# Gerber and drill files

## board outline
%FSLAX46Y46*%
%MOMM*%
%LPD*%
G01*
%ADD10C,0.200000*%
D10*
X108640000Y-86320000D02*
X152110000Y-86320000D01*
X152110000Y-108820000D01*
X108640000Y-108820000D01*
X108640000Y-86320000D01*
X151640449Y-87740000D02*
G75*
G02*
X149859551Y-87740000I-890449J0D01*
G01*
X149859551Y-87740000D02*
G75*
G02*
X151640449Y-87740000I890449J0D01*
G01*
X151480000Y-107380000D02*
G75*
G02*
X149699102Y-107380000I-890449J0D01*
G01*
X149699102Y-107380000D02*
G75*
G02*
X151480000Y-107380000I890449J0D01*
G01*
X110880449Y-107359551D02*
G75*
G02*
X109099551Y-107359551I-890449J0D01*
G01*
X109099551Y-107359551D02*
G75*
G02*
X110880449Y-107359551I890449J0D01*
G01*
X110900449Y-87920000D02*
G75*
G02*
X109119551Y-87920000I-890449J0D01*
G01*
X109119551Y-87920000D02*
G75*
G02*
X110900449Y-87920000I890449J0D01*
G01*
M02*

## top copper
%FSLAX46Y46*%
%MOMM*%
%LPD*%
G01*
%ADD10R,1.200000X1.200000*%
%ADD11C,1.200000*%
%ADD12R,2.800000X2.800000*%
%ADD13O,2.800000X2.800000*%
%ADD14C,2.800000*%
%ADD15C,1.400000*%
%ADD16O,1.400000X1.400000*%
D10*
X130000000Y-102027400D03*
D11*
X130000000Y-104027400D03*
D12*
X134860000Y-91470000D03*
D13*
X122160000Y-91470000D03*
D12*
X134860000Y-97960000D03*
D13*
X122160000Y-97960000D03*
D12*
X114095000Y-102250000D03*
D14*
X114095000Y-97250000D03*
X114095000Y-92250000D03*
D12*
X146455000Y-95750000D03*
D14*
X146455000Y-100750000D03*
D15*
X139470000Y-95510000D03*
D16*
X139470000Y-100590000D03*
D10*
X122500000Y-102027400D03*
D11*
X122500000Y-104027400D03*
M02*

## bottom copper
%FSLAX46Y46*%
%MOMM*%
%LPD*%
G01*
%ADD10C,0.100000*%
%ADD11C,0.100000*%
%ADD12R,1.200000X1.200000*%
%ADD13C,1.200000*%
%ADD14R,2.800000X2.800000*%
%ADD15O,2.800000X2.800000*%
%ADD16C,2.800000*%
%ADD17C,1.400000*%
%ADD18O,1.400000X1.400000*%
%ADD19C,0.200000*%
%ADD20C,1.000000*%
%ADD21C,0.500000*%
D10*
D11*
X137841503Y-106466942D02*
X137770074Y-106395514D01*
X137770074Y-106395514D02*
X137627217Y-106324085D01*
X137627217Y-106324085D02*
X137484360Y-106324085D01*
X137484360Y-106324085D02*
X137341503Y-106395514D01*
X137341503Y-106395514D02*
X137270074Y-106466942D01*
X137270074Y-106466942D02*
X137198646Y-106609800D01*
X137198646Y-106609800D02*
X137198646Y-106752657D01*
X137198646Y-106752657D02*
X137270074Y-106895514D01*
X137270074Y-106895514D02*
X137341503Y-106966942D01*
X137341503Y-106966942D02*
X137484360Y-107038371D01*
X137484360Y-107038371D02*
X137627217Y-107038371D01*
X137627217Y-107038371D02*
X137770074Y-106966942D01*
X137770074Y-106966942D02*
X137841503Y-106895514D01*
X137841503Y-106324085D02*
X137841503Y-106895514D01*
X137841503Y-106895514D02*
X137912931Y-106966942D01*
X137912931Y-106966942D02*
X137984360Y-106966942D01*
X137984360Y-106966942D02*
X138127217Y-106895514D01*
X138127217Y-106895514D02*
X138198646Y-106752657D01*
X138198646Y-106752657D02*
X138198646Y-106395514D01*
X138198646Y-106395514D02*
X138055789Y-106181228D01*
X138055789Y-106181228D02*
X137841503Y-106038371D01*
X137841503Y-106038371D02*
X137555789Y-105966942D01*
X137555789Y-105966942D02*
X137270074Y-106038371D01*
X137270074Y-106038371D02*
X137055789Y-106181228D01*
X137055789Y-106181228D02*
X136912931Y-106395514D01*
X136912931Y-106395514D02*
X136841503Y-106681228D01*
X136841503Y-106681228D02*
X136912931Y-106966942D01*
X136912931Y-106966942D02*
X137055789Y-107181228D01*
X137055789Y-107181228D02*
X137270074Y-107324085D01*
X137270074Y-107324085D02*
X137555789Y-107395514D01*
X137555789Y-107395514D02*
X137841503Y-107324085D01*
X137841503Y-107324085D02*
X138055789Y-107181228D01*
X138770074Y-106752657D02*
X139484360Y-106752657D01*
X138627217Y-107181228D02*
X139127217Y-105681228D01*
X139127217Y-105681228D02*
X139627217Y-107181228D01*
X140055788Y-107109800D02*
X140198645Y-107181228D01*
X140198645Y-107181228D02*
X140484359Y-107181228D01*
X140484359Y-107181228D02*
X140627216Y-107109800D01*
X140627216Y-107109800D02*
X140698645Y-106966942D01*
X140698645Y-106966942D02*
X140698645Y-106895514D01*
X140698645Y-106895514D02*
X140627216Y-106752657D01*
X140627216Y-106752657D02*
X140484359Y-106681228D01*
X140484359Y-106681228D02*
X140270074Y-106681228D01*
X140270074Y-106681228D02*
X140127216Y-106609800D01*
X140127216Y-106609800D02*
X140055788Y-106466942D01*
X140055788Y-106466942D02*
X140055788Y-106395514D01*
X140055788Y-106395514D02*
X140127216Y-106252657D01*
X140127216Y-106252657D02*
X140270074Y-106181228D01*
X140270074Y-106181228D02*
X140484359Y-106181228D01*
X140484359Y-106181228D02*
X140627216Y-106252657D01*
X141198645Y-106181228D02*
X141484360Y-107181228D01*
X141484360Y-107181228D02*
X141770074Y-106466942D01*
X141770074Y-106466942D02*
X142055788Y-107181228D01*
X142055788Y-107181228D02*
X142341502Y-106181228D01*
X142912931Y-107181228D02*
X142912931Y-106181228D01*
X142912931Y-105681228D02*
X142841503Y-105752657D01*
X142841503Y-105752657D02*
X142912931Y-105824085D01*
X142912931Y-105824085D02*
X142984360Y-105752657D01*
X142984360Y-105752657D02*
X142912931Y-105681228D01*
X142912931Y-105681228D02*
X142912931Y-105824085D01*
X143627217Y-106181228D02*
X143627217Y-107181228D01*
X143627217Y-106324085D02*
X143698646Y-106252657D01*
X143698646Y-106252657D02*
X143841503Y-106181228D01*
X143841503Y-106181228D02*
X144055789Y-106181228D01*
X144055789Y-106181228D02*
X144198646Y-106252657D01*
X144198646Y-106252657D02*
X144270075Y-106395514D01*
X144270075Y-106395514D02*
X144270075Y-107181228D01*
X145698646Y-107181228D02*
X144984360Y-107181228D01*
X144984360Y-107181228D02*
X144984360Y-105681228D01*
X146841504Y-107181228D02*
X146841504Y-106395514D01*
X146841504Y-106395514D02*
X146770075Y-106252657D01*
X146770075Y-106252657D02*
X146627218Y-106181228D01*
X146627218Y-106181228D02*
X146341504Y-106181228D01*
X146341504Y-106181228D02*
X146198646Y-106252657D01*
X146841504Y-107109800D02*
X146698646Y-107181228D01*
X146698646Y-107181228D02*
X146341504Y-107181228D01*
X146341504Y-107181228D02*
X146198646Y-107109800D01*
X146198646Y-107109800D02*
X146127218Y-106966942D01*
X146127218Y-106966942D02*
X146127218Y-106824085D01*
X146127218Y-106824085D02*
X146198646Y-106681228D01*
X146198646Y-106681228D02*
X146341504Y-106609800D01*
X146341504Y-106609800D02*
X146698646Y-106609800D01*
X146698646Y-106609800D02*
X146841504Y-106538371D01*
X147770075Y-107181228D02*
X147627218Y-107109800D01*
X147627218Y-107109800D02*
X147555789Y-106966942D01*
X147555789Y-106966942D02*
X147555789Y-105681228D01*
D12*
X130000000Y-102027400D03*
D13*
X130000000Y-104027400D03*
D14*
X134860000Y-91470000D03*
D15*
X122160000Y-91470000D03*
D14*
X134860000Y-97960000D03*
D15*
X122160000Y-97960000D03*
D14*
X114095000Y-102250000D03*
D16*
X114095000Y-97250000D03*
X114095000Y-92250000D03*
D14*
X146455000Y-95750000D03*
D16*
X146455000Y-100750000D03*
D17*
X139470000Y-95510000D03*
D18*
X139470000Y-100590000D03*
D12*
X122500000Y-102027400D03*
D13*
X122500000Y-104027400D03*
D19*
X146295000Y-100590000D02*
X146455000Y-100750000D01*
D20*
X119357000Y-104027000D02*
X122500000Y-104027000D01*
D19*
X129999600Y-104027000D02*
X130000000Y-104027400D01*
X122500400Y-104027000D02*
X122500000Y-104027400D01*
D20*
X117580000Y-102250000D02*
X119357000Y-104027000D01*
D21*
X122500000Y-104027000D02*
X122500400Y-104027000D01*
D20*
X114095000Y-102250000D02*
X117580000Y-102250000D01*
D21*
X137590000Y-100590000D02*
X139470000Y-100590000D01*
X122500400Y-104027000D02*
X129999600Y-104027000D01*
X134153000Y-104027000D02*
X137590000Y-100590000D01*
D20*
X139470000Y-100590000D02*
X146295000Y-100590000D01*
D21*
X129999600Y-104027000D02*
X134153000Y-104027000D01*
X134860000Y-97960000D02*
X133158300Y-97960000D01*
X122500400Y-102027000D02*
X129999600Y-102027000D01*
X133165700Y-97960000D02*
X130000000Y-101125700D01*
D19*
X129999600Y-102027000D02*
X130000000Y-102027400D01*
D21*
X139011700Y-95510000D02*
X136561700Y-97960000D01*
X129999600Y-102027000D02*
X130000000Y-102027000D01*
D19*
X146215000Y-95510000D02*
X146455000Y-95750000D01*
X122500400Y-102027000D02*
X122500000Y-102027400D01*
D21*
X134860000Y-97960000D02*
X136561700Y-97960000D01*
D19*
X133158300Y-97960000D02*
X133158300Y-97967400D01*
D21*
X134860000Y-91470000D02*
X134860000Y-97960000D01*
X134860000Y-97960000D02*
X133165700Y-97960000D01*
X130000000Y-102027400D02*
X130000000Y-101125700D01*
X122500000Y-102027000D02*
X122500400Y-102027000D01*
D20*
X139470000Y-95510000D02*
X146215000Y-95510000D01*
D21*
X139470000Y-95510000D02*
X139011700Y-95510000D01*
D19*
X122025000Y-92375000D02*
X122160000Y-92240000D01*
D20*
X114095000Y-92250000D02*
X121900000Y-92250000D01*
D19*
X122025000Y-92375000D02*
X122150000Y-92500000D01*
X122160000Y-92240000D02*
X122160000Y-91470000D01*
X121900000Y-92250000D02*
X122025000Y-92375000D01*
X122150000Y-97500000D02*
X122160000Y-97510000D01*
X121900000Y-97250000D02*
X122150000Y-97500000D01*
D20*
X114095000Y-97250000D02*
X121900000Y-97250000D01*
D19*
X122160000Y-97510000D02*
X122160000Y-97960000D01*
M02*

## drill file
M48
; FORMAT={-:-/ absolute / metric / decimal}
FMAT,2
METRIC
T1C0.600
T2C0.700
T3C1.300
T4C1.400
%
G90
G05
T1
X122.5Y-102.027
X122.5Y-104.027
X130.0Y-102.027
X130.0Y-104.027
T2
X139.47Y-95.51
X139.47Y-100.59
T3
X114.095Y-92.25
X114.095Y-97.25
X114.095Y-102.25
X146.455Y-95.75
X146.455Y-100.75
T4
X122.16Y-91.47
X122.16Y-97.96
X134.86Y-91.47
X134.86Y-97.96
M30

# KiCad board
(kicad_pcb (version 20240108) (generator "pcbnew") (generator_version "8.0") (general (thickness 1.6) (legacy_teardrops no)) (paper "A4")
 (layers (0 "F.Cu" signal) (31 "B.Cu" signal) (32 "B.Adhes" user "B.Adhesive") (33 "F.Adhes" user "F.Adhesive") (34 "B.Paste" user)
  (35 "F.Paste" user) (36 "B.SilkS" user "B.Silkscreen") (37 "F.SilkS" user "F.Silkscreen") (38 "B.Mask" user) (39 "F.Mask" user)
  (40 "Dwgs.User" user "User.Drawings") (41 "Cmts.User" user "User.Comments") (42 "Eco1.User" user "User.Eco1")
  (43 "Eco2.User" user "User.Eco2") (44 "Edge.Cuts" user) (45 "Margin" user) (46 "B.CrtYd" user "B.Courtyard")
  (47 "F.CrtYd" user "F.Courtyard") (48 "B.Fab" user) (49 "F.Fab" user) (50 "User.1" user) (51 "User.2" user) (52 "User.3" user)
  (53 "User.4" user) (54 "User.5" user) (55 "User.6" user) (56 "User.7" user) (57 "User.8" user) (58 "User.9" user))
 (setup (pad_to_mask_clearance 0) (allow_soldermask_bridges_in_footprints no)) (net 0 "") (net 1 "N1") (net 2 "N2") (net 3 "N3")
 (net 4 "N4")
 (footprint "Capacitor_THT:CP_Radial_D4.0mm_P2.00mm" (layer "F.Cu") (at 130 102.0274 -90)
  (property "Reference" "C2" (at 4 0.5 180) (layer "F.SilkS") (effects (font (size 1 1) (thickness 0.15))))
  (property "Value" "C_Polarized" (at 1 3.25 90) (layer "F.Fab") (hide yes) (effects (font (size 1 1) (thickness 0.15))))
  (pad "1" thru_hole rect (at 0 0 270) (size 1.2 1.2) (drill 0.6) (layers "*.Cu" "*.Mask") (remove_unused_layers no) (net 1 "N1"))
  (pad "2" thru_hole circle (at 2 0 270) (size 1.2 1.2) (drill 0.6) (layers "*.Cu" "*.Mask") (remove_unused_layers no) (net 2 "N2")))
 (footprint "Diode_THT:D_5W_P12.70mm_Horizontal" (layer "F.Cu") (at 134.86 91.47 180)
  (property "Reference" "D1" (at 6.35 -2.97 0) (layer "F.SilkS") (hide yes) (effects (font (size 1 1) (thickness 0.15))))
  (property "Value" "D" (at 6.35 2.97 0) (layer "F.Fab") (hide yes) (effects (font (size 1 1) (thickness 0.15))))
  (pad "1" thru_hole rect (at 0 0 180) (size 2.8 2.8) (drill 1.4) (layers "*.Cu" "*.Mask") (remove_unused_layers no) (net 1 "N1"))
  (pad "2" thru_hole oval (at 12.7 0 180) (size 2.8 2.8) (drill 1.4) (layers "*.Cu" "*.Mask") (remove_unused_layers no) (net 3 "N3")))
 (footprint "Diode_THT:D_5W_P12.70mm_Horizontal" (layer "F.Cu") (at 134.86 97.96 180)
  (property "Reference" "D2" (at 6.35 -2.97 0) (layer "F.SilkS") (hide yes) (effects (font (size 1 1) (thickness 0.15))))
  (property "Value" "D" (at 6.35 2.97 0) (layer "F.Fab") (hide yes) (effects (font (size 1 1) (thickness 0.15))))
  (pad "1" thru_hole rect (at 0 0 180) (size 2.8 2.8) (drill 1.4) (layers "*.Cu" "*.Mask") (remove_unused_layers no) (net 1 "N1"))
  (pad "2" thru_hole oval (at 12.7 0 180) (size 2.8 2.8) (drill 1.4) (layers "*.Cu" "*.Mask") (remove_unused_layers no) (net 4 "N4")))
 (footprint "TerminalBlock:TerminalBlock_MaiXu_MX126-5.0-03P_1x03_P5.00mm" (layer "F.Cu") (at 114.095 102.25 90)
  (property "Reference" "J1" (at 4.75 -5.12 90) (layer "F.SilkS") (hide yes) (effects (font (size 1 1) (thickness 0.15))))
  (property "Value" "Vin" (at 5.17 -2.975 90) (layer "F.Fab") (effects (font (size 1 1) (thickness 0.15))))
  (pad "1" thru_hole rect (at 0 0 90) (size 2.8 2.8) (drill 1.3) (layers "*.Cu" "*.Mask") (remove_unused_layers no) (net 2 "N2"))
  (pad "2" thru_hole circle (at 5 0 90) (size 2.8 2.8) (drill 1.3) (layers "*.Cu" "*.Mask") (remove_unused_layers no) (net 4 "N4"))
  (pad "3" thru_hole circle (at 10 0 90) (size 2.8 2.8) (drill 1.3) (layers "*.Cu" "*.Mask") (remove_unused_layers no) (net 3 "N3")))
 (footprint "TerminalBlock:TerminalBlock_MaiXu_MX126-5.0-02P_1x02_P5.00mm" (layer "F.Cu") (at 146.455 95.75 -90)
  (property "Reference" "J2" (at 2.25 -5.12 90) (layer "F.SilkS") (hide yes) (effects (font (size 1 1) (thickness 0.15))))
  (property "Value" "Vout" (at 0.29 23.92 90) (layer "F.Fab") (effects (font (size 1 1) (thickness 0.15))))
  (pad "1" thru_hole rect (at 0 0 270) (size 2.8 2.8) (drill 1.3) (layers "*.Cu" "*.Mask") (remove_unused_layers no) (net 1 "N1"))
  (pad "2" thru_hole circle (at 5 0 270) (size 2.8 2.8) (drill 1.3) (layers "*.Cu" "*.Mask") (remove_unused_layers no) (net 2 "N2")))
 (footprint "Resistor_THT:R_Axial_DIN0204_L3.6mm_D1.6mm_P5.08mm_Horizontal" (layer "F.Cu") (at 139.47 95.51 -90)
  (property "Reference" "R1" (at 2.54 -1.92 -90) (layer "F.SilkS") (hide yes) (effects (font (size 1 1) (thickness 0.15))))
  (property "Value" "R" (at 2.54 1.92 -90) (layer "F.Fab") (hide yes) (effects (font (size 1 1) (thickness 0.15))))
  (pad "1" thru_hole circle (at 0 0 270) (size 1.4 1.4) (drill 0.7) (layers "*.Cu" "*.Mask") (remove_unused_layers no) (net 1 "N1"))
  (pad "2" thru_hole oval (at 5.08 0 270) (size 1.4 1.4) (drill 0.7) (layers "*.Cu" "*.Mask") (remove_unused_layers no) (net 2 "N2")))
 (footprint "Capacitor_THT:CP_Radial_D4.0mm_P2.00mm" (layer "F.Cu") (at 122.5 102.0274 -90)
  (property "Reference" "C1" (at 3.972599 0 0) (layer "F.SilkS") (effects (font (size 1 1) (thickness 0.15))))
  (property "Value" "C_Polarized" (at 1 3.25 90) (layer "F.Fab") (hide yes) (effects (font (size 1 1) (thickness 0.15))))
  (pad "1" thru_hole rect (at 0 0 270) (size 1.2 1.2) (drill 0.6) (layers "*.Cu" "*.Mask") (remove_unused_layers no) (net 1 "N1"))
  (pad "2" thru_hole circle (at 2 0 270) (size 1.2 1.2) (drill 0.6) (layers "*.Cu" "*.Mask") (remove_unused_layers no) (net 2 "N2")))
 (gr_rect (start 108.64 86.32) (end 152.11 108.82) (stroke (width 0.2) (type default)) (fill none) (layer "Edge.Cuts"))
 (gr_circle (center 150.75 87.74) (end 151.640449 87.74) (stroke (width 0.2) (type default)) (fill none) (layer "Edge.Cuts"))
 (gr_circle (center 150.589551 107.38) (end 151.48 107.38) (stroke (width 0.2) (type default)) (fill none) (layer "Edge.Cuts"))
 (gr_circle (center 109.99 107.359551) (end 110.880449 107.359551) (stroke (width 0.2) (type default)) (fill none) (layer "Edge.Cuts"))
 (gr_circle (center 110.01 87.92) (end 110.900449 87.92) (stroke (width 0.2) (type default)) (fill none) (layer "Edge.Cuts"))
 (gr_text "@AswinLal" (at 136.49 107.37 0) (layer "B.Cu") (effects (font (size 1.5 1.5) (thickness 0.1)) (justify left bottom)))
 (segment (start 146.295 100.59) (end 146.455 100.75) (width 0.2) (layer "B.Cu") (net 2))
 (segment (start 119.357 104.027) (end 122.5 104.027) (width 1) (layer "B.Cu") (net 2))
 (segment (start 129.9996 104.027) (end 130 104.0274) (width 0.2) (layer "B.Cu") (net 2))
 (segment (start 122.5004 104.027) (end 122.5 104.0274) (width 0.2) (layer "B.Cu") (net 2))
 (segment (start 117.58 102.25) (end 119.357 104.027) (width 1) (layer "B.Cu") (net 2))
 (segment (start 122.5 104.027) (end 122.5004 104.027) (width 0.5) (layer "B.Cu") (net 2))
 (segment (start 114.095 102.25) (end 117.58 102.25) (width 1) (layer "B.Cu") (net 2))
 (segment (start 137.59 100.59) (end 139.47 100.59) (width 0.5) (layer "B.Cu") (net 2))
 (segment (start 122.5004 104.027) (end 129.9996 104.027) (width 0.5) (layer "B.Cu") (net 2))
 (segment (start 134.153 104.027) (end 137.59 100.59) (width 0.5) (layer "B.Cu") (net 2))
 (segment (start 139.47 100.59) (end 146.295 100.59) (width 1) (layer "B.Cu") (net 2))
 (segment (start 129.9996 104.027) (end 134.153 104.027) (width 0.5) (layer "B.Cu") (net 2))
 (segment (start 134.86 97.96) (end 133.1583 97.96) (width 0.5) (layer "B.Cu") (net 1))
 (segment (start 122.5004 102.027) (end 129.9996 102.027) (width 0.5) (layer "B.Cu") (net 1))
 (segment (start 133.1657 97.96) (end 130 101.1257) (width 0.5) (layer "B.Cu") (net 1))
 (segment (start 129.9996 102.027) (end 130 102.0274) (width 0.2) (layer "B.Cu") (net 1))
 (segment (start 139.0117 95.51) (end 136.5617 97.96) (width 0.5) (layer "B.Cu") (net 1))
 (segment (start 129.9996 102.027) (end 130 102.027) (width 0.5) (layer "B.Cu") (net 1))
 (segment (start 146.215 95.51) (end 146.455 95.75) (width 0.2) (layer "B.Cu") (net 1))
 (segment (start 122.5004 102.027) (end 122.5 102.0274) (width 0.2) (layer "B.Cu") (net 1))
 (segment (start 134.86 97.96) (end 136.5617 97.96) (width 0.5) (layer "B.Cu") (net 1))
 (segment (start 133.1583 97.96) (end 133.1583 97.9674) (width 0.2) (layer "B.Cu") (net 1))
 (segment (start 134.86 91.47) (end 134.86 97.96) (width 0.5) (layer "B.Cu") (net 1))
 (segment (start 134.86 97.96) (end 133.1657 97.96) (width 0.5) (layer "B.Cu") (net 1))
 (segment (start 130 102.0274) (end 130 101.1257) (width 0.5) (layer "B.Cu") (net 1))
 (segment (start 122.5 102.027) (end 122.5004 102.027) (width 0.5) (layer "B.Cu") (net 1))
 (segment (start 139.47 95.51) (end 146.215 95.51) (width 1) (layer "B.Cu") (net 1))
 (segment (start 139.47 95.51) (end 139.0117 95.51) (width 0.5) (layer "B.Cu") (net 1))
 (segment (start 122.025 92.375) (end 122.16 92.24) (width 0.2) (layer "B.Cu") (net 3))
 (segment (start 114.095 92.25) (end 121.9 92.25) (width 1) (layer "B.Cu") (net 3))
 (segment (start 122.025 92.375) (end 122.15 92.5) (width 0.2) (layer "B.Cu") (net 3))
 (segment (start 122.16 92.24) (end 122.16 91.47) (width 0.2) (layer "B.Cu") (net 3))
 (segment (start 121.9 92.25) (end 122.025 92.375) (width 0.2) (layer "B.Cu") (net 3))
 (segment (start 122.15 97.5) (end 122.16 97.51) (width 0.2) (layer "B.Cu") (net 4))
 (segment (start 121.9 97.25) (end 122.15 97.5) (width 0.2) (layer "B.Cu") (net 4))
 (segment (start 114.095 97.25) (end 121.9 97.25) (width 1) (layer "B.Cu") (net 4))
 (segment (start 122.16 97.51) (end 122.16 97.96) (width 0.2) (layer "B.Cu") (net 4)))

